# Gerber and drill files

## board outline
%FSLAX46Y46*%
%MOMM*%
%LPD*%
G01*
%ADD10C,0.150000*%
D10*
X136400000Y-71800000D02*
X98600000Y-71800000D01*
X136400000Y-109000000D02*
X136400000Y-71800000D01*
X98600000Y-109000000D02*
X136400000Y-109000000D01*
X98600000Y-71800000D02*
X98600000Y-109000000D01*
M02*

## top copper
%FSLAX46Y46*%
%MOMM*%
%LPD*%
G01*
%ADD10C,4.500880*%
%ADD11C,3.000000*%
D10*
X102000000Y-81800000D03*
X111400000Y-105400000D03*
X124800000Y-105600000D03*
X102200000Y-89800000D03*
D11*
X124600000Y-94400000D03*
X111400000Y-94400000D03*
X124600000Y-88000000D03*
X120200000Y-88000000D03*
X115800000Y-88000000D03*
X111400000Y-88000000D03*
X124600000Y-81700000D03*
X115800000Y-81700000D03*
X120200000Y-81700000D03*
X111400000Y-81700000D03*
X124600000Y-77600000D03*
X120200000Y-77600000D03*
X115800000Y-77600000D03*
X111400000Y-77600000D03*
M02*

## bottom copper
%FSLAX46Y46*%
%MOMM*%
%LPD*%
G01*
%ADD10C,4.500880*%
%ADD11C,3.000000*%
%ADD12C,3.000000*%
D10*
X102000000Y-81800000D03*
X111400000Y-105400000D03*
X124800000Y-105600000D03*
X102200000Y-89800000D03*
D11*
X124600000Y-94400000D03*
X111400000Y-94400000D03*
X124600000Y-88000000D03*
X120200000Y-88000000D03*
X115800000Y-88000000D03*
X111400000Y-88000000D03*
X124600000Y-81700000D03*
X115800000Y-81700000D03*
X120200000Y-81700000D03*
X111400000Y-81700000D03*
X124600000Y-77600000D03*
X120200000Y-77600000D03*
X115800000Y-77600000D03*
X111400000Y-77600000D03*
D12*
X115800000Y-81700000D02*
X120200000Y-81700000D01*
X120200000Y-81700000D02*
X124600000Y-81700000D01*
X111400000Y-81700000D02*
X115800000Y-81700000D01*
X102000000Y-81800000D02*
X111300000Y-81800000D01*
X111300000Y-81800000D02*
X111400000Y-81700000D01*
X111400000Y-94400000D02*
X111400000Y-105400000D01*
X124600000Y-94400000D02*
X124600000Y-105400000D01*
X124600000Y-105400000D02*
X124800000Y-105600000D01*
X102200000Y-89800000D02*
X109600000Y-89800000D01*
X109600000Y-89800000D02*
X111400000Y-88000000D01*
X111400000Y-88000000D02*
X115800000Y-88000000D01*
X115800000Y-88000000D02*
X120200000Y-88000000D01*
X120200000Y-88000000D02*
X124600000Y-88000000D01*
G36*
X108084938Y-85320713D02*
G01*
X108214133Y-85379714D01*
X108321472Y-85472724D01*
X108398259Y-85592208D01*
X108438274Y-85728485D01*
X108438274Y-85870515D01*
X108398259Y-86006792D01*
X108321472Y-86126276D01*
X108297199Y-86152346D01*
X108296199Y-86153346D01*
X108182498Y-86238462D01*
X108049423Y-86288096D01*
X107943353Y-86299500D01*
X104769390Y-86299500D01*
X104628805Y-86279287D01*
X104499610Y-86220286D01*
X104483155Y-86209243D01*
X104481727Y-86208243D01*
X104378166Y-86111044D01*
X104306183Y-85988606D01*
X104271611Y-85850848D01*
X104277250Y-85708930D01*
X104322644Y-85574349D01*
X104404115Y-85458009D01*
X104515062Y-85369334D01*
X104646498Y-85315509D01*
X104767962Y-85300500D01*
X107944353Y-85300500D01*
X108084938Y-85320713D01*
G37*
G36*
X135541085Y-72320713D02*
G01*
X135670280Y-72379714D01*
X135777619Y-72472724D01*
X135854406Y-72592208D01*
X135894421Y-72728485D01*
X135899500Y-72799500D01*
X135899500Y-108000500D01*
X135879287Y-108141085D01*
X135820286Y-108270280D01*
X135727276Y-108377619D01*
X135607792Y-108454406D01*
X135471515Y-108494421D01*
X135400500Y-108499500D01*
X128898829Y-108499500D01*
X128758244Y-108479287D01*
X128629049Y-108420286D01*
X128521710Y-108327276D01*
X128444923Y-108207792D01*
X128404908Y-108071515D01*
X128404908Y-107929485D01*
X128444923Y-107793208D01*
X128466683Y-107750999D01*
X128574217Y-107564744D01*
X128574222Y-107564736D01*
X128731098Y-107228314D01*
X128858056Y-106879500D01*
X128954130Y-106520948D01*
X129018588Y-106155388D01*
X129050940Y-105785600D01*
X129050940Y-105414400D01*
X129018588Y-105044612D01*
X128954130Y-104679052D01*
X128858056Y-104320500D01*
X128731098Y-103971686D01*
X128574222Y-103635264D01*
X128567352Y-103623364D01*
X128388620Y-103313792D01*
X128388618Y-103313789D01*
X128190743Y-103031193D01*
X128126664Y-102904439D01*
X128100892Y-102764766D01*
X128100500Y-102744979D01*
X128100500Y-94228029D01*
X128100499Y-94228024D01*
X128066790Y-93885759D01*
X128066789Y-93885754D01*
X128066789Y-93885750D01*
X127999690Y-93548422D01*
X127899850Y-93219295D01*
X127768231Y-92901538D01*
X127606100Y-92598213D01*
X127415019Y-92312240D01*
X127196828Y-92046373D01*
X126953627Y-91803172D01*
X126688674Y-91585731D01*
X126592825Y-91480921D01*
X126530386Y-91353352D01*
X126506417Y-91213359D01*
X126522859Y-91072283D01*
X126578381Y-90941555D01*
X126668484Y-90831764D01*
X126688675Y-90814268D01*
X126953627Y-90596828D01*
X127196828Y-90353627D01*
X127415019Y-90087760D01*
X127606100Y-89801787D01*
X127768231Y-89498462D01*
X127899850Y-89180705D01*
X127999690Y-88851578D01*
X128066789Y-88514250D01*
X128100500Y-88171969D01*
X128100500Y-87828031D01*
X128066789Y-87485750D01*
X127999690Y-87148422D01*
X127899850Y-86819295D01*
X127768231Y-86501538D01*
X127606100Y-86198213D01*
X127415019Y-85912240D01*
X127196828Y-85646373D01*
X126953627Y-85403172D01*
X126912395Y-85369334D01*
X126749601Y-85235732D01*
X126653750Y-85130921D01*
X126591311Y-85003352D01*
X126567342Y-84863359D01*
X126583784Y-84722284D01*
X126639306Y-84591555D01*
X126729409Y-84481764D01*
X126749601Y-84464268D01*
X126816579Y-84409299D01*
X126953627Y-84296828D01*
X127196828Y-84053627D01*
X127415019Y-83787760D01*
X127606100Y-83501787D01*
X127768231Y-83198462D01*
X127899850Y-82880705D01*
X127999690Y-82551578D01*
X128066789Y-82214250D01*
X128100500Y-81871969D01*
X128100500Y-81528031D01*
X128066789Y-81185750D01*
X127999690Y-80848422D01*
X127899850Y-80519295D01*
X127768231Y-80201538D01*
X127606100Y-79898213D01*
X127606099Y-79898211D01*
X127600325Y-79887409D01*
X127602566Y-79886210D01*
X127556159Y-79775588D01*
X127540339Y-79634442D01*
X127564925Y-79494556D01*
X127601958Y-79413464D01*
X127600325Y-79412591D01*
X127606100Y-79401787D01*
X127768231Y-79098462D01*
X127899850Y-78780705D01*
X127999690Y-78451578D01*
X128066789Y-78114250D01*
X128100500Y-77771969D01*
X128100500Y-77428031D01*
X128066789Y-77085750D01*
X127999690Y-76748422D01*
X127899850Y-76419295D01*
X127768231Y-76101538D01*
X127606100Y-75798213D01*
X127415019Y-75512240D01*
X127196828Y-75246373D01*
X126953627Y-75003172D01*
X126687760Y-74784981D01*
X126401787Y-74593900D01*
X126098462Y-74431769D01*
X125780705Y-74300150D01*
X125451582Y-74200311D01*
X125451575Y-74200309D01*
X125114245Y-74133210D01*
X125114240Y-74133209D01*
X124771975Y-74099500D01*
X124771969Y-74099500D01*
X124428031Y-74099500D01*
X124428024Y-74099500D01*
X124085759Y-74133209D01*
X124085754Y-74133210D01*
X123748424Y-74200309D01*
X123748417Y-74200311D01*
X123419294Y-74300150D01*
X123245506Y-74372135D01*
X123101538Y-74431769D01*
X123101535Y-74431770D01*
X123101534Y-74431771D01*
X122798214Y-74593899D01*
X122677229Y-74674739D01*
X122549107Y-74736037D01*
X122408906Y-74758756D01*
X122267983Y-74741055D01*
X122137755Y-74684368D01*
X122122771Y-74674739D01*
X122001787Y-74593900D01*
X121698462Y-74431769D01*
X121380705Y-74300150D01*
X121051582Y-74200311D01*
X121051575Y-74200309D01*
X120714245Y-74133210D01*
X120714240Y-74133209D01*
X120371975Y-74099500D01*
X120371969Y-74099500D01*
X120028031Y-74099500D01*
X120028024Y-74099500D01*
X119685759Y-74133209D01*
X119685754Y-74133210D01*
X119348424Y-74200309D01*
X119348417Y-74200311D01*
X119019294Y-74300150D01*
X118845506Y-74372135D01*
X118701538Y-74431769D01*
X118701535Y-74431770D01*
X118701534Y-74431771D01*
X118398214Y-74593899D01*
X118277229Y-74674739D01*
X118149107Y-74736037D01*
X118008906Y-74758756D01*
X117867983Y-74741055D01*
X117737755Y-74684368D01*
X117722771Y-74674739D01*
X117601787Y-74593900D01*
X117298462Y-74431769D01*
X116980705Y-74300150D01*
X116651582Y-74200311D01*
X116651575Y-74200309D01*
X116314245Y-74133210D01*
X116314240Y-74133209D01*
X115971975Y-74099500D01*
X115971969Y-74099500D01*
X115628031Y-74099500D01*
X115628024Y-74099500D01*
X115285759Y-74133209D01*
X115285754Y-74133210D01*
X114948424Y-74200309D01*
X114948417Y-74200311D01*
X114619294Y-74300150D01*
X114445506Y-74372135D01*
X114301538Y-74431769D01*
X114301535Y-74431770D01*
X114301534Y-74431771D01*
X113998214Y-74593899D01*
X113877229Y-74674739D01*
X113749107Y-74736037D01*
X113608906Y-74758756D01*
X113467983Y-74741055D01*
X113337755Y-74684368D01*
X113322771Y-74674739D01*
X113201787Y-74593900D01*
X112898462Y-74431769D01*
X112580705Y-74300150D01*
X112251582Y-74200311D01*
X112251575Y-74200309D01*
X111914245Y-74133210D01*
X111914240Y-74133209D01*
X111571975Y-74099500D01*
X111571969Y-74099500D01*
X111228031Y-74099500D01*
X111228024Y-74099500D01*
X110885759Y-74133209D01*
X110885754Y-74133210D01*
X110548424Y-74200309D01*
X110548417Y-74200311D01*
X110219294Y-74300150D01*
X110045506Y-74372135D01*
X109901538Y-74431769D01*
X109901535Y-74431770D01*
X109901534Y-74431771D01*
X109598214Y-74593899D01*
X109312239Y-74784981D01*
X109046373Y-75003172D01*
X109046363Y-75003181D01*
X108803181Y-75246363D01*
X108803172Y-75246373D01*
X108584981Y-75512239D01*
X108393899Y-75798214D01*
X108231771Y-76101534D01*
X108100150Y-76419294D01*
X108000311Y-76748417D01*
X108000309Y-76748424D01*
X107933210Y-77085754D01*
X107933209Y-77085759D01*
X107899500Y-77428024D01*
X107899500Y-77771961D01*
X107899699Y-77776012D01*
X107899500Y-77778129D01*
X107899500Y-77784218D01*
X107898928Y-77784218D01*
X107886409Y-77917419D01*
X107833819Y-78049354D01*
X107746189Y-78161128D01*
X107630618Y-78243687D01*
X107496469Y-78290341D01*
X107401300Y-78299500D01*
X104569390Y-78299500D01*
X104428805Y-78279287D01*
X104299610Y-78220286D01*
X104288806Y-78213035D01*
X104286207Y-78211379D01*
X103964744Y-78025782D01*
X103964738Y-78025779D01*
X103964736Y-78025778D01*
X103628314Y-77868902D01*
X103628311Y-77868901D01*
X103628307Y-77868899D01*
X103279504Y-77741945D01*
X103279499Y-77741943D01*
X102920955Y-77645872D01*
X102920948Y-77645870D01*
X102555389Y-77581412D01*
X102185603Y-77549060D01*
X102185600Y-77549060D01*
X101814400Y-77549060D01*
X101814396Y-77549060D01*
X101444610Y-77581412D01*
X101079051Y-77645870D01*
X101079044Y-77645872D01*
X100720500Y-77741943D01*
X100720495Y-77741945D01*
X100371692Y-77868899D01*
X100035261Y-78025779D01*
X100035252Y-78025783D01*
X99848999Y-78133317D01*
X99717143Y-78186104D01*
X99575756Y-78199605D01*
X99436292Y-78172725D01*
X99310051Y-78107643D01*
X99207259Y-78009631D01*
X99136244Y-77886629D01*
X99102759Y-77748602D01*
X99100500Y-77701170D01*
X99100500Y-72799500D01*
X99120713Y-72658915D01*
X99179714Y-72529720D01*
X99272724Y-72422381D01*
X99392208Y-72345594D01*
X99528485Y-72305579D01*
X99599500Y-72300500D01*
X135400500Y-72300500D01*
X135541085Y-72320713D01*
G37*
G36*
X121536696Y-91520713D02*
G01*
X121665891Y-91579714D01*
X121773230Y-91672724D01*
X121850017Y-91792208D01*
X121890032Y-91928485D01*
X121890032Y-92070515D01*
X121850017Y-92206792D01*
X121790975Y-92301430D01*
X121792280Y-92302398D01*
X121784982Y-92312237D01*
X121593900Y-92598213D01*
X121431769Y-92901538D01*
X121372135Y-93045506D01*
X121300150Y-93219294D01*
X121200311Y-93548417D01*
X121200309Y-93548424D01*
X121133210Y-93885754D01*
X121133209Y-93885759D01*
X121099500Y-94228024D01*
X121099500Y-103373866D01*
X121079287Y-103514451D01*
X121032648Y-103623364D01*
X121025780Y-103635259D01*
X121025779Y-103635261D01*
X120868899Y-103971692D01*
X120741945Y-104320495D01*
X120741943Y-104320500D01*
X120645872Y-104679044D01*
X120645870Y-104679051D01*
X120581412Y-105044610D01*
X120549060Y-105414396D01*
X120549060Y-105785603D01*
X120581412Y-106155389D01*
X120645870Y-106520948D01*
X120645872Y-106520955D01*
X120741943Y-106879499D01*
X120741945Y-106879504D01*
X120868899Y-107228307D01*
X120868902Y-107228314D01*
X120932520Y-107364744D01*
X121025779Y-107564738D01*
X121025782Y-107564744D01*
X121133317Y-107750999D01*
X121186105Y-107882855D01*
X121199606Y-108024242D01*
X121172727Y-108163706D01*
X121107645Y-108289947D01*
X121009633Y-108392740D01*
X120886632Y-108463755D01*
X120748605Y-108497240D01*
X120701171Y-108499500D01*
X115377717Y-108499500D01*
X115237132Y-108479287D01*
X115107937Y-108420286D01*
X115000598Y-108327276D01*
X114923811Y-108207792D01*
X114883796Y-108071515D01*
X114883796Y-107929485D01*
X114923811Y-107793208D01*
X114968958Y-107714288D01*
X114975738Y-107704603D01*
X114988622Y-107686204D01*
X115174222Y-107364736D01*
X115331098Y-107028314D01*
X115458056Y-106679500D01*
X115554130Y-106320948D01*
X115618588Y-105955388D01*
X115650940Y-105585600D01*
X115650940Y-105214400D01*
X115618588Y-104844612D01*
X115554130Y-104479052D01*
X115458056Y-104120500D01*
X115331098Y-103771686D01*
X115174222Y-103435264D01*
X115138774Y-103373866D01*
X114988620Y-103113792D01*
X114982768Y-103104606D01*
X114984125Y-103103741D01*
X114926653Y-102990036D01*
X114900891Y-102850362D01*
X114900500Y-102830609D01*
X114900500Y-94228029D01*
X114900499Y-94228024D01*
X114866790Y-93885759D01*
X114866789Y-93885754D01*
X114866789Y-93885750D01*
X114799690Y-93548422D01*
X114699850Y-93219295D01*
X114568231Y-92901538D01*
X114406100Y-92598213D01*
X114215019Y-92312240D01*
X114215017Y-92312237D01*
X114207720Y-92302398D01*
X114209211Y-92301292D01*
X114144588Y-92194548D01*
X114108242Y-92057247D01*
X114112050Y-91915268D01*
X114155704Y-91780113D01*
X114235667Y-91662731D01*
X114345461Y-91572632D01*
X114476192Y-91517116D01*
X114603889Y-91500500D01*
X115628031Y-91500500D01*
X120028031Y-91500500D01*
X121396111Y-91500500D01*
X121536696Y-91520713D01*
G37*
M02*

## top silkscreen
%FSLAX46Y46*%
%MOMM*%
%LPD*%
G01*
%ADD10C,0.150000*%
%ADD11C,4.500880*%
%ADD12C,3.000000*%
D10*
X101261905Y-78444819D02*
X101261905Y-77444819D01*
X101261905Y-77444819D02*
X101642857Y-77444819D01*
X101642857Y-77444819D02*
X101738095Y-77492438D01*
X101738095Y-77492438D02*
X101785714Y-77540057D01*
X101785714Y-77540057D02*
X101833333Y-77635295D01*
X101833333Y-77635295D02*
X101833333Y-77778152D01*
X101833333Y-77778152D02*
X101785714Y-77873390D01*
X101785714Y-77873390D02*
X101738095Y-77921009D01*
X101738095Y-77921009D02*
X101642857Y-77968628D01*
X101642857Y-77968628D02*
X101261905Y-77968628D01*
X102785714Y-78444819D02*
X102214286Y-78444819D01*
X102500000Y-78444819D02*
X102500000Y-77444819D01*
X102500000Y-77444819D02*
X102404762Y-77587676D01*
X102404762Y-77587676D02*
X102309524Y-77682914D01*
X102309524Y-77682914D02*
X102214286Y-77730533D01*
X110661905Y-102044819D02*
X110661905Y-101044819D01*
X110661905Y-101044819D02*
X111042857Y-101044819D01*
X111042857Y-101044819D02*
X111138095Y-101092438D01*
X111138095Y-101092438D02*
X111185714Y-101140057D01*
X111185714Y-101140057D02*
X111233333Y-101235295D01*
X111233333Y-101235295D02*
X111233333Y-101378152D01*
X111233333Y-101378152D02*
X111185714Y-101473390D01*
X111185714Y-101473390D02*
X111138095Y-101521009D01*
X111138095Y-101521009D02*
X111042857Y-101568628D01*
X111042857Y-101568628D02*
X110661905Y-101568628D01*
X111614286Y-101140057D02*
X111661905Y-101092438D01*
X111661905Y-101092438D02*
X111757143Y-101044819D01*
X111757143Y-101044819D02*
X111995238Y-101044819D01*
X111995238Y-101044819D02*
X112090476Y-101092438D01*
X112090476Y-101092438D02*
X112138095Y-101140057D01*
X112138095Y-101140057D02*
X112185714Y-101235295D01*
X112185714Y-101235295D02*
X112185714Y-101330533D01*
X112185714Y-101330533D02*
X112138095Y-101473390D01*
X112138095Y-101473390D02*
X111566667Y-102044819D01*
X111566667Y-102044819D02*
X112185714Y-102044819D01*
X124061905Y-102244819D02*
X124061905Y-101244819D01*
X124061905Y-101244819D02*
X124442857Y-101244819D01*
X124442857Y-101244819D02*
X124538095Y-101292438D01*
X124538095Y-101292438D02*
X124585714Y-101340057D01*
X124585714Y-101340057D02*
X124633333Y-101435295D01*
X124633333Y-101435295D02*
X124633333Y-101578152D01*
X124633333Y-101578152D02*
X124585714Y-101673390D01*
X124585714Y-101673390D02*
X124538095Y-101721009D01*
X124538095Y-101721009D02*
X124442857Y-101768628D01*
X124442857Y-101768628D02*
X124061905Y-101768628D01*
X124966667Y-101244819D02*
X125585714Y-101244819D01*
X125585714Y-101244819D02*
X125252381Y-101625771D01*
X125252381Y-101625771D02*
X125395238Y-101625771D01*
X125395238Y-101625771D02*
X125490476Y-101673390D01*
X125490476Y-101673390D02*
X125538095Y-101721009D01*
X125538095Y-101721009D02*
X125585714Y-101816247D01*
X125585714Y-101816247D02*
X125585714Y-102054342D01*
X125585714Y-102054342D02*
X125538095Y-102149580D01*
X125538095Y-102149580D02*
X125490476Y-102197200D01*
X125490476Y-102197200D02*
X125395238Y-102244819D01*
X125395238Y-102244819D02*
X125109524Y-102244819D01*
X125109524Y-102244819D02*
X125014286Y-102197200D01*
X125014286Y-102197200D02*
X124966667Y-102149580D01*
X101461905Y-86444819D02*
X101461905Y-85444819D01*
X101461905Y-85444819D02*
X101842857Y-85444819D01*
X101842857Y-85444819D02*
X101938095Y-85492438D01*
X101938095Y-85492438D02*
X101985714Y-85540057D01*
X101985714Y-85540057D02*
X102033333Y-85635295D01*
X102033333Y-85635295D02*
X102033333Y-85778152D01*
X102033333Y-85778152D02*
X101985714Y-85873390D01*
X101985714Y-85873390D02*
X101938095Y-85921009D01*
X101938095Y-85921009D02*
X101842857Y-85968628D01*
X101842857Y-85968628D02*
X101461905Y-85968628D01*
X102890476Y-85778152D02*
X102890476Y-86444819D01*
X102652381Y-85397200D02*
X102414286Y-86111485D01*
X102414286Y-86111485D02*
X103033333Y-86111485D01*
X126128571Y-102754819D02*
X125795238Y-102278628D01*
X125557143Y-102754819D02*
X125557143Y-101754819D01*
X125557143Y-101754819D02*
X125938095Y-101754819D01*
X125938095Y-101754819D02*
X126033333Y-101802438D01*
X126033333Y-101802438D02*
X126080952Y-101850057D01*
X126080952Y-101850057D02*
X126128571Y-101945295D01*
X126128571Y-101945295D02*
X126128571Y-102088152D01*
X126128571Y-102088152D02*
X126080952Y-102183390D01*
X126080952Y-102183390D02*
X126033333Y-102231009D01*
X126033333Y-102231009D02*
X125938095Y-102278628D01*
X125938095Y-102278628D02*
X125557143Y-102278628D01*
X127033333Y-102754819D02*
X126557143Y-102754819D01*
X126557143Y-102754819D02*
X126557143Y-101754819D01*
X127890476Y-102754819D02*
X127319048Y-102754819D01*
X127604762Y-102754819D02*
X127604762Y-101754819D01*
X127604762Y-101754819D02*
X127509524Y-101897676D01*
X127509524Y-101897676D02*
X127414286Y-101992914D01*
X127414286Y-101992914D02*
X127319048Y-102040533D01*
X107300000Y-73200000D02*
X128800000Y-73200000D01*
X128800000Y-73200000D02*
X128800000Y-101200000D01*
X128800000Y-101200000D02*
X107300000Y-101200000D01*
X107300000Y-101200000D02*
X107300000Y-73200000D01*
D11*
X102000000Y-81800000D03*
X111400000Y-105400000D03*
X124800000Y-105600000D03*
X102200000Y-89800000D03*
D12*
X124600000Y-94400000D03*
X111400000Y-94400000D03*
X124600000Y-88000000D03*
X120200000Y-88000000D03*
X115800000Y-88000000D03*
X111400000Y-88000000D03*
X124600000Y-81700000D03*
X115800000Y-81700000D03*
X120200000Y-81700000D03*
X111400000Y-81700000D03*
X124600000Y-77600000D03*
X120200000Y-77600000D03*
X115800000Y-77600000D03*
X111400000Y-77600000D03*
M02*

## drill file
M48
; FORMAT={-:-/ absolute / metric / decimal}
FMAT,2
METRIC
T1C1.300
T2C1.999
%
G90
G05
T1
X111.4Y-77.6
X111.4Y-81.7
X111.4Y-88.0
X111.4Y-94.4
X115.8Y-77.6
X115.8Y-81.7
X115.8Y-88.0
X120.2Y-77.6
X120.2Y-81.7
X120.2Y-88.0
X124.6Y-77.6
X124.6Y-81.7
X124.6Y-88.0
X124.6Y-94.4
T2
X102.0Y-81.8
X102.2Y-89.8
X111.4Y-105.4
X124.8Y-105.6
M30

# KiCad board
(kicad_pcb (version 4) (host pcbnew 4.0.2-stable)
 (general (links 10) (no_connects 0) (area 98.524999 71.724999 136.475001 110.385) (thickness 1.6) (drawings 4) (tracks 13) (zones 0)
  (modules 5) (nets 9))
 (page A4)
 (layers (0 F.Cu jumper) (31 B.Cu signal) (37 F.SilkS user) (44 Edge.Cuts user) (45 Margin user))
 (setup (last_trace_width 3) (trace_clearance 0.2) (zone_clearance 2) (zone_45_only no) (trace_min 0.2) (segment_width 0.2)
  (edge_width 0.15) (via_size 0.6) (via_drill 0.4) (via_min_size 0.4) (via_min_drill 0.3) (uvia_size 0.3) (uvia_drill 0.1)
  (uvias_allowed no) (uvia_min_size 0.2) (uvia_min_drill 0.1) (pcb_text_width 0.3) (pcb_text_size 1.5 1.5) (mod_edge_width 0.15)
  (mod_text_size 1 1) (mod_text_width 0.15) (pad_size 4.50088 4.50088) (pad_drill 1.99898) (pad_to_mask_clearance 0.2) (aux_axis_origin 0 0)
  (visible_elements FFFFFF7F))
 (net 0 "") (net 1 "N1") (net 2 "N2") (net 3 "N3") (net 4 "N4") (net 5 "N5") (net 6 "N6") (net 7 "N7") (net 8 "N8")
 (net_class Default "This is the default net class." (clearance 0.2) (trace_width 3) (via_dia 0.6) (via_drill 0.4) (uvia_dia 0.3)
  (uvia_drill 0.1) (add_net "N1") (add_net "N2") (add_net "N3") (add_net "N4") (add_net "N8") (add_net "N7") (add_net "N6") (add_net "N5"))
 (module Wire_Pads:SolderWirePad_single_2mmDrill (layer F.Cu) (at 102 81.8)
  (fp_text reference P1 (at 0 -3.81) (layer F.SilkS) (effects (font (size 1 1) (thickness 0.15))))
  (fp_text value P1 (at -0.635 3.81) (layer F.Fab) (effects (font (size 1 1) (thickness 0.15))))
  (pad 1 thru_hole circle (at 0 0) (size 4.50088 4.50088) (drill 1.99898) (layers *.Cu *.Mask F.SilkS) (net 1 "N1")))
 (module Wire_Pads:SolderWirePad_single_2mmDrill (layer F.Cu) (at 111.4 105.4)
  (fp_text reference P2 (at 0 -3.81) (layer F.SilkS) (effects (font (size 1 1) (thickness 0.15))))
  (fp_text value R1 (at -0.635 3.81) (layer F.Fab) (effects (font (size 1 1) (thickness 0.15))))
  (pad 1 thru_hole circle (at 0 0) (size 4.50088 4.50088) (drill 1.99898) (layers *.Cu *.Mask F.SilkS) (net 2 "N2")))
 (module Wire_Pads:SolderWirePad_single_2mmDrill (layer F.Cu) (at 124.8 105.6)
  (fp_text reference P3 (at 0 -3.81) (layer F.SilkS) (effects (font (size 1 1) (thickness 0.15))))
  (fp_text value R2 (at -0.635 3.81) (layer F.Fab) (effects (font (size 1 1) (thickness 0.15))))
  (pad 1 thru_hole circle (at 0 0) (size 4.50088 4.50088) (drill 1.99898) (layers *.Cu *.Mask F.SilkS) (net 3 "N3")))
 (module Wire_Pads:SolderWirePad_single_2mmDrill (layer F.Cu) (at 102.2 89.8)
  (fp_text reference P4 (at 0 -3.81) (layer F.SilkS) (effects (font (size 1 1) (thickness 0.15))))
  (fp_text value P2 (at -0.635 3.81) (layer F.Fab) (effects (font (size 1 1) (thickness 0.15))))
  (pad 1 thru_hole circle (at 0 0) (size 4.50088 4.50088) (drill 1.99898) (layers *.Cu *.Mask F.SilkS) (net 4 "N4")))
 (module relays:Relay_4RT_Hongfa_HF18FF (layer F.Cu) (at 111.4 77.6)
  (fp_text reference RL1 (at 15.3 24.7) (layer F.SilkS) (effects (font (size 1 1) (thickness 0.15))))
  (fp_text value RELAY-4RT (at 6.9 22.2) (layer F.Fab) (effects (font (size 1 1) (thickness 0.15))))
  (fp_line (start -4.1 -4.4) (end 17.4 -4.4) (layer F.SilkS) (width 0.15))
  (fp_line (start 17.4 -4.4) (end 17.4 23.6) (layer F.SilkS) (width 0.15))
  (fp_line (start 17.4 23.6) (end -4.1 23.6) (layer F.SilkS) (width 0.15))
  (fp_line (start -4.1 23.6) (end -4.1 -4.4) (layer F.SilkS) (width 0.15))
  (pad 14 thru_hole circle (at 13.2 16.8) (size 3 3) (drill 1.3) (layers *.Cu *.Mask F.SilkS) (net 3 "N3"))
  (pad 13 thru_hole circle (at 0 16.8) (size 3 3) (drill 1.3) (layers *.Cu *.Mask F.SilkS) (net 2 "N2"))
  (pad 12 thru_hole circle (at 13.2 10.4) (size 3 3) (drill 1.3) (layers *.Cu *.Mask F.SilkS) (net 4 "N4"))
  (pad 11 thru_hole circle (at 8.8 10.4) (size 3 3) (drill 1.3) (layers *.Cu *.Mask F.SilkS) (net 4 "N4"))
  (pad 10 thru_hole circle (at 4.4 10.4) (size 3 3) (drill 1.3) (layers *.Cu *.Mask F.SilkS) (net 4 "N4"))
  (pad 9 thru_hole circle (at 0 10.4) (size 3 3) (drill 1.3) (layers *.Cu *.Mask F.SilkS) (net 4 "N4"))
  (pad 8 thru_hole circle (at 13.2 4.1) (size 3 3) (drill 1.3) (layers *.Cu *.Mask F.SilkS) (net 1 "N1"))
  (pad 6 thru_hole circle (at 4.4 4.1) (size 3 3) (drill 1.3) (layers *.Cu *.Mask F.SilkS) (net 1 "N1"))
  (pad 7 thru_hole circle (at 8.8 4.1) (size 3 3) (drill 1.3) (layers *.Cu *.Mask F.SilkS) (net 1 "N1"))
  (pad 5 thru_hole circle (at 0 4.1) (size 3 3) (drill 1.3) (layers *.Cu *.Mask F.SilkS) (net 1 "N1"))
  (pad 4 thru_hole circle (at 13.2 0) (size 3 3) (drill 1.3) (layers *.Cu *.Mask F.SilkS) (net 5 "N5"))
  (pad 3 thru_hole circle (at 8.8 0) (size 3 3) (drill 1.3) (layers *.Cu *.Mask F.SilkS) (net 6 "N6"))
  (pad 2 thru_hole circle (at 4.4 0) (size 3 3) (drill 1.3) (layers *.Cu *.Mask F.SilkS) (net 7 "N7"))
  (pad 1 thru_hole circle (at 0 0) (size 3 3) (drill 1.3) (layers *.Cu *.Mask F.SilkS) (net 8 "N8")))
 (gr_line (start 136.4 71.8) (end 98.6 71.8) (angle 90) (layer Edge.Cuts) (width 0.15))
 (gr_line (start 136.4 109) (end 136.4 71.8) (angle 90) (layer Edge.Cuts) (width 0.15))
 (gr_line (start 98.6 109) (end 136.4 109) (angle 90) (layer Edge.Cuts) (width 0.15))
 (gr_line (start 98.6 71.8) (end 98.6 109) (angle 90) (layer Edge.Cuts) (width 0.15))
 (segment (start 115.8 81.7) (end 120.2 81.7) (width 3) (layer B.Cu) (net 1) (status C00000))
 (segment (start 120.2 81.7) (end 124.6 81.7) (width 3) (layer B.Cu) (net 1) (status C00000))
 (segment (start 111.4 81.7) (end 115.8 81.7) (width 3) (layer B.Cu) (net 1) (status C00000))
 (segment (start 102 81.8) (end 111.3 81.8) (width 3) (layer B.Cu) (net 1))
 (segment (start 111.3 81.8) (end 111.4 81.7) (width 3) (layer B.Cu) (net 1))
 (segment (start 111.4 94.4) (end 111.4 105.4) (width 3) (layer B.Cu) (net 2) (status C00000))
 (segment (start 124.6 94.4) (end 124.6 105.4) (width 3) (layer B.Cu) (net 3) (status C00000))
 (segment (start 124.6 105.4) (end 124.8 105.6) (width 3) (layer B.Cu) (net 3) (status C00000))
 (segment (start 102.2 89.8) (end 109.6 89.8) (width 3) (layer B.Cu) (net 4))
 (segment (start 109.6 89.8) (end 111.4 88) (width 3) (layer B.Cu) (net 4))
 (segment (start 111.4 88) (end 115.8 88) (width 3) (layer B.Cu) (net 4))
 (segment (start 115.8 88) (end 120.2 88) (width 3) (layer B.Cu) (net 4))
 (segment (start 120.2 88) (end 124.6 88) (width 3) (layer B.Cu) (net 4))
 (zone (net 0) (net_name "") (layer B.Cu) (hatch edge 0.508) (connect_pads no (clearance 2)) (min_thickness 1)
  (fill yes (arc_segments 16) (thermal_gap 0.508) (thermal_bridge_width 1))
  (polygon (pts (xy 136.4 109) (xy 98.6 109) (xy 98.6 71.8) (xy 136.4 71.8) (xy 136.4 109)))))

